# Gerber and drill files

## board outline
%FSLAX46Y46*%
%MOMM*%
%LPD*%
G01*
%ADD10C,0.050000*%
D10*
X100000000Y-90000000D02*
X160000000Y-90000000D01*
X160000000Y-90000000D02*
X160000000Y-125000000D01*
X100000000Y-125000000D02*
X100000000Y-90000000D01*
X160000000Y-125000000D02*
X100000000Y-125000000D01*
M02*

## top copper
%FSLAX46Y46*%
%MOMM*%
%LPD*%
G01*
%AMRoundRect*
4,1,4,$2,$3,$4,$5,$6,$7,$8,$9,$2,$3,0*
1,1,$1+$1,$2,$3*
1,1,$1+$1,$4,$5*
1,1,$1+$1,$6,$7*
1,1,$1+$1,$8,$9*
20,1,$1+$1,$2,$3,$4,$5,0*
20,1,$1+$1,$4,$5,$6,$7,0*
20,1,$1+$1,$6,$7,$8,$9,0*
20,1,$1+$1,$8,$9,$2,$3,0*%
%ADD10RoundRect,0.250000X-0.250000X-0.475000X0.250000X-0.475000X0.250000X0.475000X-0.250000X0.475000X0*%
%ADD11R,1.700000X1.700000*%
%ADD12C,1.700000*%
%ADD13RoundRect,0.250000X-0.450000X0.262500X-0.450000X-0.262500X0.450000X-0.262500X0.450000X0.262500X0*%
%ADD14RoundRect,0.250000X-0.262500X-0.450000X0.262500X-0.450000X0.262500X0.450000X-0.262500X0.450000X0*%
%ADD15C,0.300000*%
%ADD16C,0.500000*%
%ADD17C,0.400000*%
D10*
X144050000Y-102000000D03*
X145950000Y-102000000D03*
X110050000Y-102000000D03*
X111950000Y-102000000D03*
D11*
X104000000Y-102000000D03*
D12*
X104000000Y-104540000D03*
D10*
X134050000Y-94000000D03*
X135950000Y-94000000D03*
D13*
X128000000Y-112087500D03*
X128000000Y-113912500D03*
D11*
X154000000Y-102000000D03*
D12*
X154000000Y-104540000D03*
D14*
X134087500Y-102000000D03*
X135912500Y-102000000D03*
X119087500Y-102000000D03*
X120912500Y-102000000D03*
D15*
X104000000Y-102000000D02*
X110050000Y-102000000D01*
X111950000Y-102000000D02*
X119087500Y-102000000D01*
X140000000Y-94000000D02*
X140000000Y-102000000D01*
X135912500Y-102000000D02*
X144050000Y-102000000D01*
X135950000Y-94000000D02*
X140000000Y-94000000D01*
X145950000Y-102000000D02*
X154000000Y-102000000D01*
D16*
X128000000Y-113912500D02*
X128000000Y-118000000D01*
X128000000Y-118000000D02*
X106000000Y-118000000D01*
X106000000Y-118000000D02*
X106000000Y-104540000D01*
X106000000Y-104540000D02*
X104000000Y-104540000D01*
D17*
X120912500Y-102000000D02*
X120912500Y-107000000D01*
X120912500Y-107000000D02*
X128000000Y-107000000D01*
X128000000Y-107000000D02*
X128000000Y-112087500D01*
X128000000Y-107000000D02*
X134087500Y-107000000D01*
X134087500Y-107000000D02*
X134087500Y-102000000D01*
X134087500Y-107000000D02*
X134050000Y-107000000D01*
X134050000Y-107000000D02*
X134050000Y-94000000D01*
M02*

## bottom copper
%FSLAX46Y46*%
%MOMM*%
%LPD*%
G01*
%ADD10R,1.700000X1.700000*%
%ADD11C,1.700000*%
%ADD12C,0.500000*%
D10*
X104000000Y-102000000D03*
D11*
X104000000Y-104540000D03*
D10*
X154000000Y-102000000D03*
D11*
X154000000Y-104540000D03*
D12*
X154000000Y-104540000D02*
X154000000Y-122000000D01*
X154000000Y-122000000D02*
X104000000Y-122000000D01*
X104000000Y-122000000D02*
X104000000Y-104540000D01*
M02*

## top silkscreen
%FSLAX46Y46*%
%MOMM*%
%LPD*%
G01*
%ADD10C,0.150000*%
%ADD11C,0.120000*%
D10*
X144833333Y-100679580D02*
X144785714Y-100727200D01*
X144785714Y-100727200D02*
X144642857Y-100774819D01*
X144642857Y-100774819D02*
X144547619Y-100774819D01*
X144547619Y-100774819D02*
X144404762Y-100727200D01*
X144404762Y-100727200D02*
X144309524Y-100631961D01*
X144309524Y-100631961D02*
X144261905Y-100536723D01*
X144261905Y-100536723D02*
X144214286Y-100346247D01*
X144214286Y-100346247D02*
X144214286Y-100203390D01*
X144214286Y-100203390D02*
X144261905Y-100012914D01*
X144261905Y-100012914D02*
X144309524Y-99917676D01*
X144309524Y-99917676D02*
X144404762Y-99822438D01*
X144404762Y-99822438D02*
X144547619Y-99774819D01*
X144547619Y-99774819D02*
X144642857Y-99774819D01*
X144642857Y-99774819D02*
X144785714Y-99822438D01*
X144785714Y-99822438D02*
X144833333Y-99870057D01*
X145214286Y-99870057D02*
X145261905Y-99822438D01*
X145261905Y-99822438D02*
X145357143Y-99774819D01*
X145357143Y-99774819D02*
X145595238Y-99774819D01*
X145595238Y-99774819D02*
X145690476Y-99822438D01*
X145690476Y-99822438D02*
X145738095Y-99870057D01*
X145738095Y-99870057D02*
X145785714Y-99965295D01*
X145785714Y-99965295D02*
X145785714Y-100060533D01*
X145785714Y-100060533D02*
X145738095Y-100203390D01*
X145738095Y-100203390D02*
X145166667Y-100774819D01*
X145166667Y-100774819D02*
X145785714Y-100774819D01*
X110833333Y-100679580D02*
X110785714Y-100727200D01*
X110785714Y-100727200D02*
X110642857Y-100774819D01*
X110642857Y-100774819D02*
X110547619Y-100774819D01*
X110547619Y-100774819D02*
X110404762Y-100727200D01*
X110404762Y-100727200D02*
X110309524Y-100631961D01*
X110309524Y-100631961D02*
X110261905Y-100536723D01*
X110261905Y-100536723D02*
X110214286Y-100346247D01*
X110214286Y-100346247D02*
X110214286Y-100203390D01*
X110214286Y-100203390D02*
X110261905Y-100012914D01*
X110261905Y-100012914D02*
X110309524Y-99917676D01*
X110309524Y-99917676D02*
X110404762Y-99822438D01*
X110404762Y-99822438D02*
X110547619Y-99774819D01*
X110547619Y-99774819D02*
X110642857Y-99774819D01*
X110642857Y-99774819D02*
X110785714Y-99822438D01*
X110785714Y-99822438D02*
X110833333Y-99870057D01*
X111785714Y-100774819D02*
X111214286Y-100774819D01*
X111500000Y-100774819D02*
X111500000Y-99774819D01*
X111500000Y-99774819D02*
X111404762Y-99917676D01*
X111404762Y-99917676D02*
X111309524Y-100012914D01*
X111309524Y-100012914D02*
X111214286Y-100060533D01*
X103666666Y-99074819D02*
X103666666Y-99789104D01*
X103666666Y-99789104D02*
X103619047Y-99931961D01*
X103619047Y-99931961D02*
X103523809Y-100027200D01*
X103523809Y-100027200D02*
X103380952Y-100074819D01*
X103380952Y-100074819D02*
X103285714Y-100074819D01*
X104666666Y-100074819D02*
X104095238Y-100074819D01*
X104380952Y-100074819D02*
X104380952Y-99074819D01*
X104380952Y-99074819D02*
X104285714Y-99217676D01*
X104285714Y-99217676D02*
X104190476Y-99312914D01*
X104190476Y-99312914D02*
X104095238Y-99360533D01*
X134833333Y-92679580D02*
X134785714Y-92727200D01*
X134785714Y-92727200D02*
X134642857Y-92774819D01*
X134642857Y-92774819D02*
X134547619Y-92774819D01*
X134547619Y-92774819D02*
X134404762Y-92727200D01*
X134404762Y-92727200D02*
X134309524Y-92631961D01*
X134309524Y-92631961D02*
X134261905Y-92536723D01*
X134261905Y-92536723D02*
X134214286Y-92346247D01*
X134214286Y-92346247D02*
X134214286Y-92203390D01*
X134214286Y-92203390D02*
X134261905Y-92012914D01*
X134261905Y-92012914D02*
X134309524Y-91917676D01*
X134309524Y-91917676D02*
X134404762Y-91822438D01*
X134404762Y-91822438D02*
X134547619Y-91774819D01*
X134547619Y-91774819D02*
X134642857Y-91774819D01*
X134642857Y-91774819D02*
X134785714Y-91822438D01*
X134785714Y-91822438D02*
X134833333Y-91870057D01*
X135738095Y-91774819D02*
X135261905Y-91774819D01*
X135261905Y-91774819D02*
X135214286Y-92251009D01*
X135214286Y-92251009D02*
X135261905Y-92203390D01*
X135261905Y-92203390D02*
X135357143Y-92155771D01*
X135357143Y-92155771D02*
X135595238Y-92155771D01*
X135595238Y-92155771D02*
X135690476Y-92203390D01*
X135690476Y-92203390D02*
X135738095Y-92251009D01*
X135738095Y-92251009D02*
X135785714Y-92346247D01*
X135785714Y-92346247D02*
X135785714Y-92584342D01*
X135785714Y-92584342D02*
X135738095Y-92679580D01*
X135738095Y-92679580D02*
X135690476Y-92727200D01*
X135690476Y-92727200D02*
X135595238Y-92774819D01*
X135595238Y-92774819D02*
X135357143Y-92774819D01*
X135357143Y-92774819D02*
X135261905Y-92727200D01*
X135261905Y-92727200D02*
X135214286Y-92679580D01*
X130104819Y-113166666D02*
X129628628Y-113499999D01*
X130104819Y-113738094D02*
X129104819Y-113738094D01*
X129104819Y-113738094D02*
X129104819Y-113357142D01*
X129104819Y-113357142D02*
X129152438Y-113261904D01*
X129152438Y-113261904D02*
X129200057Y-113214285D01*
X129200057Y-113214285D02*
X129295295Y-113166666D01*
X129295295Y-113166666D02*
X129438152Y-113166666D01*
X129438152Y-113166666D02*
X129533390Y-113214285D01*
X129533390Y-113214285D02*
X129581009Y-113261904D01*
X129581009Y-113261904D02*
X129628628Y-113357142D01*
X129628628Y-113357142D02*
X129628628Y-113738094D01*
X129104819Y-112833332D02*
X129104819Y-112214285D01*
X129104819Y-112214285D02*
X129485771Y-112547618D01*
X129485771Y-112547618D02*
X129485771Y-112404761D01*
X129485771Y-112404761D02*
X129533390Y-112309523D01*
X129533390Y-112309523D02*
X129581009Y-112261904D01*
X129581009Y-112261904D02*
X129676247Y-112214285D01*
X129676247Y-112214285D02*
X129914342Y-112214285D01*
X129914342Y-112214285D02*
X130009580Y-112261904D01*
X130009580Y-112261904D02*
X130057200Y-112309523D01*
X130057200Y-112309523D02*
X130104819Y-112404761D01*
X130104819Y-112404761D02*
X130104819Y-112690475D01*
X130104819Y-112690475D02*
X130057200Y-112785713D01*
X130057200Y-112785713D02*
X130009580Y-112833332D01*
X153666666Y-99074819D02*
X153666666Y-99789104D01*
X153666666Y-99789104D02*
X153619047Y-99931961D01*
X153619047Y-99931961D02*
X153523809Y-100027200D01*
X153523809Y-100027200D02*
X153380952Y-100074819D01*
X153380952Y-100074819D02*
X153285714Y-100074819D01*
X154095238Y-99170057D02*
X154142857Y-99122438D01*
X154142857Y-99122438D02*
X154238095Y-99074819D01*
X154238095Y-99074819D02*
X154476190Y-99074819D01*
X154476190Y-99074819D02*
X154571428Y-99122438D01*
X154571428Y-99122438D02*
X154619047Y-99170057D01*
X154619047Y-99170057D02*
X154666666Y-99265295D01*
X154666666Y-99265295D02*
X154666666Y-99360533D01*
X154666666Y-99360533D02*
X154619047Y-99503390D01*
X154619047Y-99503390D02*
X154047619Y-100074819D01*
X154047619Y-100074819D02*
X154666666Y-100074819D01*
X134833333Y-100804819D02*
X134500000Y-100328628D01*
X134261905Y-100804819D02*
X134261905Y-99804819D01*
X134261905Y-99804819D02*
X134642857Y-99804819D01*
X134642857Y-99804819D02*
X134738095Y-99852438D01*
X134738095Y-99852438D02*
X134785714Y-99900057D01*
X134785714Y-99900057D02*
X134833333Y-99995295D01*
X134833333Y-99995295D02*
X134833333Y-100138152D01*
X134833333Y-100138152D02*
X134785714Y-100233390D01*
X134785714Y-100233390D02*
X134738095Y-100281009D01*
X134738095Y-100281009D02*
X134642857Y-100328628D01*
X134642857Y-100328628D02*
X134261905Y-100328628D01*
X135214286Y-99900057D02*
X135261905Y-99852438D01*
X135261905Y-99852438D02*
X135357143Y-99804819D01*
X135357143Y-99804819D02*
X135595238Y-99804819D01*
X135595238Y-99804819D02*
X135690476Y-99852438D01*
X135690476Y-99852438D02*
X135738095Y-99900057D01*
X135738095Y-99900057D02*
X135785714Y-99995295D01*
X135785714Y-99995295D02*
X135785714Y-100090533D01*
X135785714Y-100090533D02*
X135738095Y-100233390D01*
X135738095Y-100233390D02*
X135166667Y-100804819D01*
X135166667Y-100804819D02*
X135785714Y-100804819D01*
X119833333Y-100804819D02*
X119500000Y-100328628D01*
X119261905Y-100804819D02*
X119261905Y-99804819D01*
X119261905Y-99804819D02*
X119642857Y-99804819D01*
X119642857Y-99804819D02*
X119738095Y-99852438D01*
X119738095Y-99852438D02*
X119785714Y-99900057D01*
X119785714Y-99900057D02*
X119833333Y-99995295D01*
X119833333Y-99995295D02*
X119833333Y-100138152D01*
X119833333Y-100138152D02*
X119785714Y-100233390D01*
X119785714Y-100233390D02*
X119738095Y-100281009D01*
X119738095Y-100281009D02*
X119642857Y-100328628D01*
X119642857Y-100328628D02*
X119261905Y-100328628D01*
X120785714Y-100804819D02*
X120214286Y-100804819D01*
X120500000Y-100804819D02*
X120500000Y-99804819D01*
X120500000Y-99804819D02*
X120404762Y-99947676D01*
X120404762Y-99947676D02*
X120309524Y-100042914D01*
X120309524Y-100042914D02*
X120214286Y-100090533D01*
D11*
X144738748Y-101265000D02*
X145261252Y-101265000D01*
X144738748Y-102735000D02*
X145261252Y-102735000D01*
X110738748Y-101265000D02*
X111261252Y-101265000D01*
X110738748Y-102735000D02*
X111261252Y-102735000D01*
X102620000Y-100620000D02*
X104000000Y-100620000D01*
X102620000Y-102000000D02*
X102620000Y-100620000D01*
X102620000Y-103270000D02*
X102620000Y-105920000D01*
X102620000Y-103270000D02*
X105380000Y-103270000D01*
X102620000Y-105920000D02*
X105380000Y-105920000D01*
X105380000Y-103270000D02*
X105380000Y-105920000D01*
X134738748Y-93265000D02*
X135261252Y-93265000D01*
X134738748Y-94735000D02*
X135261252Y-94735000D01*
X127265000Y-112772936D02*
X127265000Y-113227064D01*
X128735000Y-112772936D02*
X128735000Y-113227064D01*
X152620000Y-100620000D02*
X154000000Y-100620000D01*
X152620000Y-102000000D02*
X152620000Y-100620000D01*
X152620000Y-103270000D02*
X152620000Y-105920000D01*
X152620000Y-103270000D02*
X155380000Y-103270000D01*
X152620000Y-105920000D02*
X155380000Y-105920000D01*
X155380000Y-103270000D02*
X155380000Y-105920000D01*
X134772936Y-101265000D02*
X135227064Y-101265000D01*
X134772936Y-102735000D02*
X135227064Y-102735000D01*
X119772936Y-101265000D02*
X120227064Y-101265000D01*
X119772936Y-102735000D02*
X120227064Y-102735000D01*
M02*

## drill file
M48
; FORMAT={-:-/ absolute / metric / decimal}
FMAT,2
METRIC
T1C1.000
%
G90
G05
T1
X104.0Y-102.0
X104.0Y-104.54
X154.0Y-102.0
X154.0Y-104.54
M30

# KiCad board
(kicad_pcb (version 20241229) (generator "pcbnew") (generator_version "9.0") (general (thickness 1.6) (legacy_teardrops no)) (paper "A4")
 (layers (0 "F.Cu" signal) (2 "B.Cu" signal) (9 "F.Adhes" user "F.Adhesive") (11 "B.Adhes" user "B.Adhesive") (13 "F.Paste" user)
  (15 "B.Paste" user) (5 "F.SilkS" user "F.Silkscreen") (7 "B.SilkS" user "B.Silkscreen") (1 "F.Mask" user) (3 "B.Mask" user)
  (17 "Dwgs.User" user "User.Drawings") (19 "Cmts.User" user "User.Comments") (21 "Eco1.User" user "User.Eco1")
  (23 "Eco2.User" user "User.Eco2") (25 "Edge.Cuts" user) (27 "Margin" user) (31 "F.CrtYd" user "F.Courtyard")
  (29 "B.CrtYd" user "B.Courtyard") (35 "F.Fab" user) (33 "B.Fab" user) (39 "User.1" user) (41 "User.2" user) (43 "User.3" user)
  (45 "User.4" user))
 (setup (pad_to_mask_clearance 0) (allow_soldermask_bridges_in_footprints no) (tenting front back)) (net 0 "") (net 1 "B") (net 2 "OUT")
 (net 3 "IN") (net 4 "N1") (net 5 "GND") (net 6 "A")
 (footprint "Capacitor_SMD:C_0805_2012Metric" (layer "F.Cu") (at 145 102)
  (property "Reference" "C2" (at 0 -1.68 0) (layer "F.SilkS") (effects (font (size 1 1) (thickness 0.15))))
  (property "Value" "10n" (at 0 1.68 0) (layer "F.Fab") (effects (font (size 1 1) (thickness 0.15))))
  (fp_line (start -0.261252 -0.735) (end 0.261252 -0.735) (stroke (width 0.12) (type solid)) (layer "F.SilkS"))
  (fp_line (start -0.261252 0.735) (end 0.261252 0.735) (stroke (width 0.12) (type solid)) (layer "F.SilkS"))
  (pad "1" smd roundrect (at -0.95 0) (size 1 1.45) (layers "F.Cu" "F.Mask" "F.Paste") (roundrect_rratio 0.25) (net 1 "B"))
  (pad "2" smd roundrect (at 0.95 0) (size 1 1.45) (layers "F.Cu" "F.Mask" "F.Paste") (roundrect_rratio 0.25) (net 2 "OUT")))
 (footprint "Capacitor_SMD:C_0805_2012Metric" (layer "F.Cu") (at 111 102)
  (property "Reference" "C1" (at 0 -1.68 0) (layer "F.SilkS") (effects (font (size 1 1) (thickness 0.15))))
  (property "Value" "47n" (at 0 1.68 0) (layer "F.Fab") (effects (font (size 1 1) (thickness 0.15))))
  (fp_line (start -0.261252 -0.735) (end 0.261252 -0.735) (stroke (width 0.12) (type solid)) (layer "F.SilkS"))
  (fp_line (start -0.261252 0.735) (end 0.261252 0.735) (stroke (width 0.12) (type solid)) (layer "F.SilkS"))
  (pad "1" smd roundrect (at -0.95 0) (size 1 1.45) (layers "F.Cu" "F.Mask" "F.Paste") (roundrect_rratio 0.25) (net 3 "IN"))
  (pad "2" smd roundrect (at 0.95 0) (size 1 1.45) (layers "F.Cu" "F.Mask" "F.Paste") (roundrect_rratio 0.25) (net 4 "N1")))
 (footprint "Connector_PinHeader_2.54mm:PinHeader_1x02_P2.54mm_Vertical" (layer "F.Cu") (at 104 102)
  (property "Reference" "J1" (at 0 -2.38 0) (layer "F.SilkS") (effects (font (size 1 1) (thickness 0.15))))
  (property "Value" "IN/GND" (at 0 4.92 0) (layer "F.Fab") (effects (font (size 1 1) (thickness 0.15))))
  (fp_line (start -1.38 -1.38) (end 0 -1.38) (stroke (width 0.12) (type solid)) (layer "F.SilkS"))
  (fp_line (start -1.38 0) (end -1.38 -1.38) (stroke (width 0.12) (type solid)) (layer "F.SilkS"))
  (fp_line (start -1.38 1.27) (end -1.38 3.92) (stroke (width 0.12) (type solid)) (layer "F.SilkS"))
  (fp_line (start -1.38 1.27) (end 1.38 1.27) (stroke (width 0.12) (type solid)) (layer "F.SilkS"))
  (fp_line (start -1.38 3.92) (end 1.38 3.92) (stroke (width 0.12) (type solid)) (layer "F.SilkS"))
  (fp_line (start 1.38 1.27) (end 1.38 3.92) (stroke (width 0.12) (type solid)) (layer "F.SilkS"))
  (pad "1" thru_hole rect (at 0 0) (size 1.7 1.7) (drill 1) (layers "*.Cu" "*.Mask") (remove_unused_layers no) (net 3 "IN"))
  (pad "2" thru_hole circle (at 0 2.54) (size 1.7 1.7) (drill 1) (layers "*.Cu" "*.Mask") (remove_unused_layers no) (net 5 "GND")))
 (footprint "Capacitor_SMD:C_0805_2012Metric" (layer "F.Cu") (at 135 94)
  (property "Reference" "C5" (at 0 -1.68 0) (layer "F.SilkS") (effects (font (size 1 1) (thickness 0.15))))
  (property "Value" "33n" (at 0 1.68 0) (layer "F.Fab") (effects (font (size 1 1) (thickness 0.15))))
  (fp_line (start -0.261252 -0.735) (end 0.261252 -0.735) (stroke (width 0.12) (type solid)) (layer "F.SilkS"))
  (fp_line (start -0.261252 0.735) (end 0.261252 0.735) (stroke (width 0.12) (type solid)) (layer "F.SilkS"))
  (pad "1" smd roundrect (at -0.95 0) (size 1 1.45) (layers "F.Cu" "F.Mask" "F.Paste") (roundrect_rratio 0.25) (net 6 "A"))
  (pad "2" smd roundrect (at 0.95 0) (size 1 1.45) (layers "F.Cu" "F.Mask" "F.Paste") (roundrect_rratio 0.25) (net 1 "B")))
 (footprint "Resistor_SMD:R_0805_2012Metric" (layer "F.Cu") (at 128 113 -90)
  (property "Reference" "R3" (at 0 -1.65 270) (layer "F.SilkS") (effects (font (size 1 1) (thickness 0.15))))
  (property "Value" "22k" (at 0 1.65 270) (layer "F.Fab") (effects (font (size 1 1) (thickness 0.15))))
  (fp_line (start -0.227064 0.735) (end 0.227064 0.735) (stroke (width 0.12) (type solid)) (layer "F.SilkS"))
  (fp_line (start -0.227064 -0.735) (end 0.227064 -0.735) (stroke (width 0.12) (type solid)) (layer "F.SilkS"))
  (pad "1" smd roundrect (at -0.9125 0 270) (size 1.025 1.4) (layers "F.Cu" "F.Mask" "F.Paste") (roundrect_rratio 0.243902) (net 6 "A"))
  (pad "2" smd roundrect (at 0.9125 0 270) (size 1.025 1.4) (layers "F.Cu" "F.Mask" "F.Paste") (roundrect_rratio 0.243902) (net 5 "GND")))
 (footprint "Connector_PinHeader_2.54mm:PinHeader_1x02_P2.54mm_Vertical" (layer "F.Cu") (at 154 102)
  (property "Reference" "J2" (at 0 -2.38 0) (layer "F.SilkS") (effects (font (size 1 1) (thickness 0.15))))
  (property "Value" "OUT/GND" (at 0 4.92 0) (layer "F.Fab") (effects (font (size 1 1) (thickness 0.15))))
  (fp_line (start -1.38 -1.38) (end 0 -1.38) (stroke (width 0.12) (type solid)) (layer "F.SilkS"))
  (fp_line (start -1.38 0) (end -1.38 -1.38) (stroke (width 0.12) (type solid)) (layer "F.SilkS"))
  (fp_line (start -1.38 1.27) (end -1.38 3.92) (stroke (width 0.12) (type solid)) (layer "F.SilkS"))
  (fp_line (start -1.38 1.27) (end 1.38 1.27) (stroke (width 0.12) (type solid)) (layer "F.SilkS"))
  (fp_line (start -1.38 3.92) (end 1.38 3.92) (stroke (width 0.12) (type solid)) (layer "F.SilkS"))
  (fp_line (start 1.38 1.27) (end 1.38 3.92) (stroke (width 0.12) (type solid)) (layer "F.SilkS"))
  (pad "1" thru_hole rect (at 0 0) (size 1.7 1.7) (drill 1) (layers "*.Cu" "*.Mask") (remove_unused_layers no) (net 2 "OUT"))
  (pad "2" thru_hole circle (at 0 2.54) (size 1.7 1.7) (drill 1) (layers "*.Cu" "*.Mask") (remove_unused_layers no) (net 5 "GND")))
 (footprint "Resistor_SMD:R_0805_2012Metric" (layer "F.Cu") (at 135 102)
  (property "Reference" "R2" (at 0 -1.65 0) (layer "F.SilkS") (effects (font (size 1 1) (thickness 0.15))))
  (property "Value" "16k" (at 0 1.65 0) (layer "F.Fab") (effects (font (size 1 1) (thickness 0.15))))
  (fp_line (start -0.227064 -0.735) (end 0.227064 -0.735) (stroke (width 0.12) (type solid)) (layer "F.SilkS"))
  (fp_line (start -0.227064 0.735) (end 0.227064 0.735) (stroke (width 0.12) (type solid)) (layer "F.SilkS"))
  (pad "1" smd roundrect (at -0.9125 0) (size 1.025 1.4) (layers "F.Cu" "F.Mask" "F.Paste") (roundrect_rratio 0.243902) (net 6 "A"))
  (pad "2" smd roundrect (at 0.9125 0) (size 1.025 1.4) (layers "F.Cu" "F.Mask" "F.Paste") (roundrect_rratio 0.243902) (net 1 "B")))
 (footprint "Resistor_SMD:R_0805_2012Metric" (layer "F.Cu") (at 120 102)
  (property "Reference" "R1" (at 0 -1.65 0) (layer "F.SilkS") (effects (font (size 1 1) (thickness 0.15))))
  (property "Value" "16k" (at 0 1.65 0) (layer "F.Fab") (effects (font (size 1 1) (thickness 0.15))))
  (fp_line (start -0.227064 -0.735) (end 0.227064 -0.735) (stroke (width 0.12) (type solid)) (layer "F.SilkS"))
  (fp_line (start -0.227064 0.735) (end 0.227064 0.735) (stroke (width 0.12) (type solid)) (layer "F.SilkS"))
  (pad "1" smd roundrect (at -0.9125 0) (size 1.025 1.4) (layers "F.Cu" "F.Mask" "F.Paste") (roundrect_rratio 0.243902) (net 4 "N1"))
  (pad "2" smd roundrect (at 0.9125 0) (size 1.025 1.4) (layers "F.Cu" "F.Mask" "F.Paste") (roundrect_rratio 0.243902) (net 6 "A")))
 (gr_line (start 100 90) (end 160 90) (stroke (width 0.05) (type default)) (layer "Edge.Cuts"))
 (gr_line (start 160 90) (end 160 125) (stroke (width 0.05) (type default)) (layer "Edge.Cuts"))
 (gr_line (start 100 125) (end 100 90) (stroke (width 0.05) (type default)) (layer "Edge.Cuts"))
 (gr_line (start 160 125) (end 100 125) (stroke (width 0.05) (type default)) (layer "Edge.Cuts"))
 (segment (start 104 102) (end 110.05 102) (width 0.3) (layer "F.Cu") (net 3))
 (segment (start 111.95 102) (end 119.0875 102) (width 0.3) (layer "F.Cu") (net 4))
 (segment (start 140 94) (end 140 102) (width 0.3) (layer "F.Cu") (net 1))
 (segment (start 135.9125 102) (end 144.05 102) (width 0.3) (layer "F.Cu") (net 1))
 (segment (start 135.95 94) (end 140 94) (width 0.3) (layer "F.Cu") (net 1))
 (segment (start 145.95 102) (end 154 102) (width 0.3) (layer "F.Cu") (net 2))
 (segment (start 128 113.9125) (end 128 118) (width 0.5) (layer "F.Cu") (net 5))
 (segment (start 128 118) (end 106 118) (width 0.5) (layer "F.Cu") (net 5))
 (segment (start 106 118) (end 106 104.54) (width 0.5) (layer "F.Cu") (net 5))
 (segment (start 106 104.54) (end 104 104.54) (width 0.5) (layer "F.Cu") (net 5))
 (segment (start 154 104.54) (end 154 122) (width 0.5) (layer "B.Cu") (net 5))
 (segment (start 154 122) (end 104 122) (width 0.5) (layer "B.Cu") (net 5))
 (segment (start 104 122) (end 104 104.54) (width 0.5) (layer "B.Cu") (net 5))
 (segment (start 120.9125 102) (end 120.9125 107) (width 0.4) (layer "F.Cu") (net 6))
 (segment (start 120.9125 107) (end 128 107) (width 0.4) (layer "F.Cu") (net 6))
 (segment (start 128 107) (end 128 112.0875) (width 0.4) (layer "F.Cu") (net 6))
 (segment (start 128 107) (end 134.0875 107) (width 0.4) (layer "F.Cu") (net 6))
 (segment (start 134.0875 107) (end 134.0875 102) (width 0.4) (layer "F.Cu") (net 6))
 (segment (start 134.0875 107) (end 134.05 107) (width 0.4) (layer "F.Cu") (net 6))
 (segment (start 134.05 107) (end 134.05 94) (width 0.4) (layer "F.Cu") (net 6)))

